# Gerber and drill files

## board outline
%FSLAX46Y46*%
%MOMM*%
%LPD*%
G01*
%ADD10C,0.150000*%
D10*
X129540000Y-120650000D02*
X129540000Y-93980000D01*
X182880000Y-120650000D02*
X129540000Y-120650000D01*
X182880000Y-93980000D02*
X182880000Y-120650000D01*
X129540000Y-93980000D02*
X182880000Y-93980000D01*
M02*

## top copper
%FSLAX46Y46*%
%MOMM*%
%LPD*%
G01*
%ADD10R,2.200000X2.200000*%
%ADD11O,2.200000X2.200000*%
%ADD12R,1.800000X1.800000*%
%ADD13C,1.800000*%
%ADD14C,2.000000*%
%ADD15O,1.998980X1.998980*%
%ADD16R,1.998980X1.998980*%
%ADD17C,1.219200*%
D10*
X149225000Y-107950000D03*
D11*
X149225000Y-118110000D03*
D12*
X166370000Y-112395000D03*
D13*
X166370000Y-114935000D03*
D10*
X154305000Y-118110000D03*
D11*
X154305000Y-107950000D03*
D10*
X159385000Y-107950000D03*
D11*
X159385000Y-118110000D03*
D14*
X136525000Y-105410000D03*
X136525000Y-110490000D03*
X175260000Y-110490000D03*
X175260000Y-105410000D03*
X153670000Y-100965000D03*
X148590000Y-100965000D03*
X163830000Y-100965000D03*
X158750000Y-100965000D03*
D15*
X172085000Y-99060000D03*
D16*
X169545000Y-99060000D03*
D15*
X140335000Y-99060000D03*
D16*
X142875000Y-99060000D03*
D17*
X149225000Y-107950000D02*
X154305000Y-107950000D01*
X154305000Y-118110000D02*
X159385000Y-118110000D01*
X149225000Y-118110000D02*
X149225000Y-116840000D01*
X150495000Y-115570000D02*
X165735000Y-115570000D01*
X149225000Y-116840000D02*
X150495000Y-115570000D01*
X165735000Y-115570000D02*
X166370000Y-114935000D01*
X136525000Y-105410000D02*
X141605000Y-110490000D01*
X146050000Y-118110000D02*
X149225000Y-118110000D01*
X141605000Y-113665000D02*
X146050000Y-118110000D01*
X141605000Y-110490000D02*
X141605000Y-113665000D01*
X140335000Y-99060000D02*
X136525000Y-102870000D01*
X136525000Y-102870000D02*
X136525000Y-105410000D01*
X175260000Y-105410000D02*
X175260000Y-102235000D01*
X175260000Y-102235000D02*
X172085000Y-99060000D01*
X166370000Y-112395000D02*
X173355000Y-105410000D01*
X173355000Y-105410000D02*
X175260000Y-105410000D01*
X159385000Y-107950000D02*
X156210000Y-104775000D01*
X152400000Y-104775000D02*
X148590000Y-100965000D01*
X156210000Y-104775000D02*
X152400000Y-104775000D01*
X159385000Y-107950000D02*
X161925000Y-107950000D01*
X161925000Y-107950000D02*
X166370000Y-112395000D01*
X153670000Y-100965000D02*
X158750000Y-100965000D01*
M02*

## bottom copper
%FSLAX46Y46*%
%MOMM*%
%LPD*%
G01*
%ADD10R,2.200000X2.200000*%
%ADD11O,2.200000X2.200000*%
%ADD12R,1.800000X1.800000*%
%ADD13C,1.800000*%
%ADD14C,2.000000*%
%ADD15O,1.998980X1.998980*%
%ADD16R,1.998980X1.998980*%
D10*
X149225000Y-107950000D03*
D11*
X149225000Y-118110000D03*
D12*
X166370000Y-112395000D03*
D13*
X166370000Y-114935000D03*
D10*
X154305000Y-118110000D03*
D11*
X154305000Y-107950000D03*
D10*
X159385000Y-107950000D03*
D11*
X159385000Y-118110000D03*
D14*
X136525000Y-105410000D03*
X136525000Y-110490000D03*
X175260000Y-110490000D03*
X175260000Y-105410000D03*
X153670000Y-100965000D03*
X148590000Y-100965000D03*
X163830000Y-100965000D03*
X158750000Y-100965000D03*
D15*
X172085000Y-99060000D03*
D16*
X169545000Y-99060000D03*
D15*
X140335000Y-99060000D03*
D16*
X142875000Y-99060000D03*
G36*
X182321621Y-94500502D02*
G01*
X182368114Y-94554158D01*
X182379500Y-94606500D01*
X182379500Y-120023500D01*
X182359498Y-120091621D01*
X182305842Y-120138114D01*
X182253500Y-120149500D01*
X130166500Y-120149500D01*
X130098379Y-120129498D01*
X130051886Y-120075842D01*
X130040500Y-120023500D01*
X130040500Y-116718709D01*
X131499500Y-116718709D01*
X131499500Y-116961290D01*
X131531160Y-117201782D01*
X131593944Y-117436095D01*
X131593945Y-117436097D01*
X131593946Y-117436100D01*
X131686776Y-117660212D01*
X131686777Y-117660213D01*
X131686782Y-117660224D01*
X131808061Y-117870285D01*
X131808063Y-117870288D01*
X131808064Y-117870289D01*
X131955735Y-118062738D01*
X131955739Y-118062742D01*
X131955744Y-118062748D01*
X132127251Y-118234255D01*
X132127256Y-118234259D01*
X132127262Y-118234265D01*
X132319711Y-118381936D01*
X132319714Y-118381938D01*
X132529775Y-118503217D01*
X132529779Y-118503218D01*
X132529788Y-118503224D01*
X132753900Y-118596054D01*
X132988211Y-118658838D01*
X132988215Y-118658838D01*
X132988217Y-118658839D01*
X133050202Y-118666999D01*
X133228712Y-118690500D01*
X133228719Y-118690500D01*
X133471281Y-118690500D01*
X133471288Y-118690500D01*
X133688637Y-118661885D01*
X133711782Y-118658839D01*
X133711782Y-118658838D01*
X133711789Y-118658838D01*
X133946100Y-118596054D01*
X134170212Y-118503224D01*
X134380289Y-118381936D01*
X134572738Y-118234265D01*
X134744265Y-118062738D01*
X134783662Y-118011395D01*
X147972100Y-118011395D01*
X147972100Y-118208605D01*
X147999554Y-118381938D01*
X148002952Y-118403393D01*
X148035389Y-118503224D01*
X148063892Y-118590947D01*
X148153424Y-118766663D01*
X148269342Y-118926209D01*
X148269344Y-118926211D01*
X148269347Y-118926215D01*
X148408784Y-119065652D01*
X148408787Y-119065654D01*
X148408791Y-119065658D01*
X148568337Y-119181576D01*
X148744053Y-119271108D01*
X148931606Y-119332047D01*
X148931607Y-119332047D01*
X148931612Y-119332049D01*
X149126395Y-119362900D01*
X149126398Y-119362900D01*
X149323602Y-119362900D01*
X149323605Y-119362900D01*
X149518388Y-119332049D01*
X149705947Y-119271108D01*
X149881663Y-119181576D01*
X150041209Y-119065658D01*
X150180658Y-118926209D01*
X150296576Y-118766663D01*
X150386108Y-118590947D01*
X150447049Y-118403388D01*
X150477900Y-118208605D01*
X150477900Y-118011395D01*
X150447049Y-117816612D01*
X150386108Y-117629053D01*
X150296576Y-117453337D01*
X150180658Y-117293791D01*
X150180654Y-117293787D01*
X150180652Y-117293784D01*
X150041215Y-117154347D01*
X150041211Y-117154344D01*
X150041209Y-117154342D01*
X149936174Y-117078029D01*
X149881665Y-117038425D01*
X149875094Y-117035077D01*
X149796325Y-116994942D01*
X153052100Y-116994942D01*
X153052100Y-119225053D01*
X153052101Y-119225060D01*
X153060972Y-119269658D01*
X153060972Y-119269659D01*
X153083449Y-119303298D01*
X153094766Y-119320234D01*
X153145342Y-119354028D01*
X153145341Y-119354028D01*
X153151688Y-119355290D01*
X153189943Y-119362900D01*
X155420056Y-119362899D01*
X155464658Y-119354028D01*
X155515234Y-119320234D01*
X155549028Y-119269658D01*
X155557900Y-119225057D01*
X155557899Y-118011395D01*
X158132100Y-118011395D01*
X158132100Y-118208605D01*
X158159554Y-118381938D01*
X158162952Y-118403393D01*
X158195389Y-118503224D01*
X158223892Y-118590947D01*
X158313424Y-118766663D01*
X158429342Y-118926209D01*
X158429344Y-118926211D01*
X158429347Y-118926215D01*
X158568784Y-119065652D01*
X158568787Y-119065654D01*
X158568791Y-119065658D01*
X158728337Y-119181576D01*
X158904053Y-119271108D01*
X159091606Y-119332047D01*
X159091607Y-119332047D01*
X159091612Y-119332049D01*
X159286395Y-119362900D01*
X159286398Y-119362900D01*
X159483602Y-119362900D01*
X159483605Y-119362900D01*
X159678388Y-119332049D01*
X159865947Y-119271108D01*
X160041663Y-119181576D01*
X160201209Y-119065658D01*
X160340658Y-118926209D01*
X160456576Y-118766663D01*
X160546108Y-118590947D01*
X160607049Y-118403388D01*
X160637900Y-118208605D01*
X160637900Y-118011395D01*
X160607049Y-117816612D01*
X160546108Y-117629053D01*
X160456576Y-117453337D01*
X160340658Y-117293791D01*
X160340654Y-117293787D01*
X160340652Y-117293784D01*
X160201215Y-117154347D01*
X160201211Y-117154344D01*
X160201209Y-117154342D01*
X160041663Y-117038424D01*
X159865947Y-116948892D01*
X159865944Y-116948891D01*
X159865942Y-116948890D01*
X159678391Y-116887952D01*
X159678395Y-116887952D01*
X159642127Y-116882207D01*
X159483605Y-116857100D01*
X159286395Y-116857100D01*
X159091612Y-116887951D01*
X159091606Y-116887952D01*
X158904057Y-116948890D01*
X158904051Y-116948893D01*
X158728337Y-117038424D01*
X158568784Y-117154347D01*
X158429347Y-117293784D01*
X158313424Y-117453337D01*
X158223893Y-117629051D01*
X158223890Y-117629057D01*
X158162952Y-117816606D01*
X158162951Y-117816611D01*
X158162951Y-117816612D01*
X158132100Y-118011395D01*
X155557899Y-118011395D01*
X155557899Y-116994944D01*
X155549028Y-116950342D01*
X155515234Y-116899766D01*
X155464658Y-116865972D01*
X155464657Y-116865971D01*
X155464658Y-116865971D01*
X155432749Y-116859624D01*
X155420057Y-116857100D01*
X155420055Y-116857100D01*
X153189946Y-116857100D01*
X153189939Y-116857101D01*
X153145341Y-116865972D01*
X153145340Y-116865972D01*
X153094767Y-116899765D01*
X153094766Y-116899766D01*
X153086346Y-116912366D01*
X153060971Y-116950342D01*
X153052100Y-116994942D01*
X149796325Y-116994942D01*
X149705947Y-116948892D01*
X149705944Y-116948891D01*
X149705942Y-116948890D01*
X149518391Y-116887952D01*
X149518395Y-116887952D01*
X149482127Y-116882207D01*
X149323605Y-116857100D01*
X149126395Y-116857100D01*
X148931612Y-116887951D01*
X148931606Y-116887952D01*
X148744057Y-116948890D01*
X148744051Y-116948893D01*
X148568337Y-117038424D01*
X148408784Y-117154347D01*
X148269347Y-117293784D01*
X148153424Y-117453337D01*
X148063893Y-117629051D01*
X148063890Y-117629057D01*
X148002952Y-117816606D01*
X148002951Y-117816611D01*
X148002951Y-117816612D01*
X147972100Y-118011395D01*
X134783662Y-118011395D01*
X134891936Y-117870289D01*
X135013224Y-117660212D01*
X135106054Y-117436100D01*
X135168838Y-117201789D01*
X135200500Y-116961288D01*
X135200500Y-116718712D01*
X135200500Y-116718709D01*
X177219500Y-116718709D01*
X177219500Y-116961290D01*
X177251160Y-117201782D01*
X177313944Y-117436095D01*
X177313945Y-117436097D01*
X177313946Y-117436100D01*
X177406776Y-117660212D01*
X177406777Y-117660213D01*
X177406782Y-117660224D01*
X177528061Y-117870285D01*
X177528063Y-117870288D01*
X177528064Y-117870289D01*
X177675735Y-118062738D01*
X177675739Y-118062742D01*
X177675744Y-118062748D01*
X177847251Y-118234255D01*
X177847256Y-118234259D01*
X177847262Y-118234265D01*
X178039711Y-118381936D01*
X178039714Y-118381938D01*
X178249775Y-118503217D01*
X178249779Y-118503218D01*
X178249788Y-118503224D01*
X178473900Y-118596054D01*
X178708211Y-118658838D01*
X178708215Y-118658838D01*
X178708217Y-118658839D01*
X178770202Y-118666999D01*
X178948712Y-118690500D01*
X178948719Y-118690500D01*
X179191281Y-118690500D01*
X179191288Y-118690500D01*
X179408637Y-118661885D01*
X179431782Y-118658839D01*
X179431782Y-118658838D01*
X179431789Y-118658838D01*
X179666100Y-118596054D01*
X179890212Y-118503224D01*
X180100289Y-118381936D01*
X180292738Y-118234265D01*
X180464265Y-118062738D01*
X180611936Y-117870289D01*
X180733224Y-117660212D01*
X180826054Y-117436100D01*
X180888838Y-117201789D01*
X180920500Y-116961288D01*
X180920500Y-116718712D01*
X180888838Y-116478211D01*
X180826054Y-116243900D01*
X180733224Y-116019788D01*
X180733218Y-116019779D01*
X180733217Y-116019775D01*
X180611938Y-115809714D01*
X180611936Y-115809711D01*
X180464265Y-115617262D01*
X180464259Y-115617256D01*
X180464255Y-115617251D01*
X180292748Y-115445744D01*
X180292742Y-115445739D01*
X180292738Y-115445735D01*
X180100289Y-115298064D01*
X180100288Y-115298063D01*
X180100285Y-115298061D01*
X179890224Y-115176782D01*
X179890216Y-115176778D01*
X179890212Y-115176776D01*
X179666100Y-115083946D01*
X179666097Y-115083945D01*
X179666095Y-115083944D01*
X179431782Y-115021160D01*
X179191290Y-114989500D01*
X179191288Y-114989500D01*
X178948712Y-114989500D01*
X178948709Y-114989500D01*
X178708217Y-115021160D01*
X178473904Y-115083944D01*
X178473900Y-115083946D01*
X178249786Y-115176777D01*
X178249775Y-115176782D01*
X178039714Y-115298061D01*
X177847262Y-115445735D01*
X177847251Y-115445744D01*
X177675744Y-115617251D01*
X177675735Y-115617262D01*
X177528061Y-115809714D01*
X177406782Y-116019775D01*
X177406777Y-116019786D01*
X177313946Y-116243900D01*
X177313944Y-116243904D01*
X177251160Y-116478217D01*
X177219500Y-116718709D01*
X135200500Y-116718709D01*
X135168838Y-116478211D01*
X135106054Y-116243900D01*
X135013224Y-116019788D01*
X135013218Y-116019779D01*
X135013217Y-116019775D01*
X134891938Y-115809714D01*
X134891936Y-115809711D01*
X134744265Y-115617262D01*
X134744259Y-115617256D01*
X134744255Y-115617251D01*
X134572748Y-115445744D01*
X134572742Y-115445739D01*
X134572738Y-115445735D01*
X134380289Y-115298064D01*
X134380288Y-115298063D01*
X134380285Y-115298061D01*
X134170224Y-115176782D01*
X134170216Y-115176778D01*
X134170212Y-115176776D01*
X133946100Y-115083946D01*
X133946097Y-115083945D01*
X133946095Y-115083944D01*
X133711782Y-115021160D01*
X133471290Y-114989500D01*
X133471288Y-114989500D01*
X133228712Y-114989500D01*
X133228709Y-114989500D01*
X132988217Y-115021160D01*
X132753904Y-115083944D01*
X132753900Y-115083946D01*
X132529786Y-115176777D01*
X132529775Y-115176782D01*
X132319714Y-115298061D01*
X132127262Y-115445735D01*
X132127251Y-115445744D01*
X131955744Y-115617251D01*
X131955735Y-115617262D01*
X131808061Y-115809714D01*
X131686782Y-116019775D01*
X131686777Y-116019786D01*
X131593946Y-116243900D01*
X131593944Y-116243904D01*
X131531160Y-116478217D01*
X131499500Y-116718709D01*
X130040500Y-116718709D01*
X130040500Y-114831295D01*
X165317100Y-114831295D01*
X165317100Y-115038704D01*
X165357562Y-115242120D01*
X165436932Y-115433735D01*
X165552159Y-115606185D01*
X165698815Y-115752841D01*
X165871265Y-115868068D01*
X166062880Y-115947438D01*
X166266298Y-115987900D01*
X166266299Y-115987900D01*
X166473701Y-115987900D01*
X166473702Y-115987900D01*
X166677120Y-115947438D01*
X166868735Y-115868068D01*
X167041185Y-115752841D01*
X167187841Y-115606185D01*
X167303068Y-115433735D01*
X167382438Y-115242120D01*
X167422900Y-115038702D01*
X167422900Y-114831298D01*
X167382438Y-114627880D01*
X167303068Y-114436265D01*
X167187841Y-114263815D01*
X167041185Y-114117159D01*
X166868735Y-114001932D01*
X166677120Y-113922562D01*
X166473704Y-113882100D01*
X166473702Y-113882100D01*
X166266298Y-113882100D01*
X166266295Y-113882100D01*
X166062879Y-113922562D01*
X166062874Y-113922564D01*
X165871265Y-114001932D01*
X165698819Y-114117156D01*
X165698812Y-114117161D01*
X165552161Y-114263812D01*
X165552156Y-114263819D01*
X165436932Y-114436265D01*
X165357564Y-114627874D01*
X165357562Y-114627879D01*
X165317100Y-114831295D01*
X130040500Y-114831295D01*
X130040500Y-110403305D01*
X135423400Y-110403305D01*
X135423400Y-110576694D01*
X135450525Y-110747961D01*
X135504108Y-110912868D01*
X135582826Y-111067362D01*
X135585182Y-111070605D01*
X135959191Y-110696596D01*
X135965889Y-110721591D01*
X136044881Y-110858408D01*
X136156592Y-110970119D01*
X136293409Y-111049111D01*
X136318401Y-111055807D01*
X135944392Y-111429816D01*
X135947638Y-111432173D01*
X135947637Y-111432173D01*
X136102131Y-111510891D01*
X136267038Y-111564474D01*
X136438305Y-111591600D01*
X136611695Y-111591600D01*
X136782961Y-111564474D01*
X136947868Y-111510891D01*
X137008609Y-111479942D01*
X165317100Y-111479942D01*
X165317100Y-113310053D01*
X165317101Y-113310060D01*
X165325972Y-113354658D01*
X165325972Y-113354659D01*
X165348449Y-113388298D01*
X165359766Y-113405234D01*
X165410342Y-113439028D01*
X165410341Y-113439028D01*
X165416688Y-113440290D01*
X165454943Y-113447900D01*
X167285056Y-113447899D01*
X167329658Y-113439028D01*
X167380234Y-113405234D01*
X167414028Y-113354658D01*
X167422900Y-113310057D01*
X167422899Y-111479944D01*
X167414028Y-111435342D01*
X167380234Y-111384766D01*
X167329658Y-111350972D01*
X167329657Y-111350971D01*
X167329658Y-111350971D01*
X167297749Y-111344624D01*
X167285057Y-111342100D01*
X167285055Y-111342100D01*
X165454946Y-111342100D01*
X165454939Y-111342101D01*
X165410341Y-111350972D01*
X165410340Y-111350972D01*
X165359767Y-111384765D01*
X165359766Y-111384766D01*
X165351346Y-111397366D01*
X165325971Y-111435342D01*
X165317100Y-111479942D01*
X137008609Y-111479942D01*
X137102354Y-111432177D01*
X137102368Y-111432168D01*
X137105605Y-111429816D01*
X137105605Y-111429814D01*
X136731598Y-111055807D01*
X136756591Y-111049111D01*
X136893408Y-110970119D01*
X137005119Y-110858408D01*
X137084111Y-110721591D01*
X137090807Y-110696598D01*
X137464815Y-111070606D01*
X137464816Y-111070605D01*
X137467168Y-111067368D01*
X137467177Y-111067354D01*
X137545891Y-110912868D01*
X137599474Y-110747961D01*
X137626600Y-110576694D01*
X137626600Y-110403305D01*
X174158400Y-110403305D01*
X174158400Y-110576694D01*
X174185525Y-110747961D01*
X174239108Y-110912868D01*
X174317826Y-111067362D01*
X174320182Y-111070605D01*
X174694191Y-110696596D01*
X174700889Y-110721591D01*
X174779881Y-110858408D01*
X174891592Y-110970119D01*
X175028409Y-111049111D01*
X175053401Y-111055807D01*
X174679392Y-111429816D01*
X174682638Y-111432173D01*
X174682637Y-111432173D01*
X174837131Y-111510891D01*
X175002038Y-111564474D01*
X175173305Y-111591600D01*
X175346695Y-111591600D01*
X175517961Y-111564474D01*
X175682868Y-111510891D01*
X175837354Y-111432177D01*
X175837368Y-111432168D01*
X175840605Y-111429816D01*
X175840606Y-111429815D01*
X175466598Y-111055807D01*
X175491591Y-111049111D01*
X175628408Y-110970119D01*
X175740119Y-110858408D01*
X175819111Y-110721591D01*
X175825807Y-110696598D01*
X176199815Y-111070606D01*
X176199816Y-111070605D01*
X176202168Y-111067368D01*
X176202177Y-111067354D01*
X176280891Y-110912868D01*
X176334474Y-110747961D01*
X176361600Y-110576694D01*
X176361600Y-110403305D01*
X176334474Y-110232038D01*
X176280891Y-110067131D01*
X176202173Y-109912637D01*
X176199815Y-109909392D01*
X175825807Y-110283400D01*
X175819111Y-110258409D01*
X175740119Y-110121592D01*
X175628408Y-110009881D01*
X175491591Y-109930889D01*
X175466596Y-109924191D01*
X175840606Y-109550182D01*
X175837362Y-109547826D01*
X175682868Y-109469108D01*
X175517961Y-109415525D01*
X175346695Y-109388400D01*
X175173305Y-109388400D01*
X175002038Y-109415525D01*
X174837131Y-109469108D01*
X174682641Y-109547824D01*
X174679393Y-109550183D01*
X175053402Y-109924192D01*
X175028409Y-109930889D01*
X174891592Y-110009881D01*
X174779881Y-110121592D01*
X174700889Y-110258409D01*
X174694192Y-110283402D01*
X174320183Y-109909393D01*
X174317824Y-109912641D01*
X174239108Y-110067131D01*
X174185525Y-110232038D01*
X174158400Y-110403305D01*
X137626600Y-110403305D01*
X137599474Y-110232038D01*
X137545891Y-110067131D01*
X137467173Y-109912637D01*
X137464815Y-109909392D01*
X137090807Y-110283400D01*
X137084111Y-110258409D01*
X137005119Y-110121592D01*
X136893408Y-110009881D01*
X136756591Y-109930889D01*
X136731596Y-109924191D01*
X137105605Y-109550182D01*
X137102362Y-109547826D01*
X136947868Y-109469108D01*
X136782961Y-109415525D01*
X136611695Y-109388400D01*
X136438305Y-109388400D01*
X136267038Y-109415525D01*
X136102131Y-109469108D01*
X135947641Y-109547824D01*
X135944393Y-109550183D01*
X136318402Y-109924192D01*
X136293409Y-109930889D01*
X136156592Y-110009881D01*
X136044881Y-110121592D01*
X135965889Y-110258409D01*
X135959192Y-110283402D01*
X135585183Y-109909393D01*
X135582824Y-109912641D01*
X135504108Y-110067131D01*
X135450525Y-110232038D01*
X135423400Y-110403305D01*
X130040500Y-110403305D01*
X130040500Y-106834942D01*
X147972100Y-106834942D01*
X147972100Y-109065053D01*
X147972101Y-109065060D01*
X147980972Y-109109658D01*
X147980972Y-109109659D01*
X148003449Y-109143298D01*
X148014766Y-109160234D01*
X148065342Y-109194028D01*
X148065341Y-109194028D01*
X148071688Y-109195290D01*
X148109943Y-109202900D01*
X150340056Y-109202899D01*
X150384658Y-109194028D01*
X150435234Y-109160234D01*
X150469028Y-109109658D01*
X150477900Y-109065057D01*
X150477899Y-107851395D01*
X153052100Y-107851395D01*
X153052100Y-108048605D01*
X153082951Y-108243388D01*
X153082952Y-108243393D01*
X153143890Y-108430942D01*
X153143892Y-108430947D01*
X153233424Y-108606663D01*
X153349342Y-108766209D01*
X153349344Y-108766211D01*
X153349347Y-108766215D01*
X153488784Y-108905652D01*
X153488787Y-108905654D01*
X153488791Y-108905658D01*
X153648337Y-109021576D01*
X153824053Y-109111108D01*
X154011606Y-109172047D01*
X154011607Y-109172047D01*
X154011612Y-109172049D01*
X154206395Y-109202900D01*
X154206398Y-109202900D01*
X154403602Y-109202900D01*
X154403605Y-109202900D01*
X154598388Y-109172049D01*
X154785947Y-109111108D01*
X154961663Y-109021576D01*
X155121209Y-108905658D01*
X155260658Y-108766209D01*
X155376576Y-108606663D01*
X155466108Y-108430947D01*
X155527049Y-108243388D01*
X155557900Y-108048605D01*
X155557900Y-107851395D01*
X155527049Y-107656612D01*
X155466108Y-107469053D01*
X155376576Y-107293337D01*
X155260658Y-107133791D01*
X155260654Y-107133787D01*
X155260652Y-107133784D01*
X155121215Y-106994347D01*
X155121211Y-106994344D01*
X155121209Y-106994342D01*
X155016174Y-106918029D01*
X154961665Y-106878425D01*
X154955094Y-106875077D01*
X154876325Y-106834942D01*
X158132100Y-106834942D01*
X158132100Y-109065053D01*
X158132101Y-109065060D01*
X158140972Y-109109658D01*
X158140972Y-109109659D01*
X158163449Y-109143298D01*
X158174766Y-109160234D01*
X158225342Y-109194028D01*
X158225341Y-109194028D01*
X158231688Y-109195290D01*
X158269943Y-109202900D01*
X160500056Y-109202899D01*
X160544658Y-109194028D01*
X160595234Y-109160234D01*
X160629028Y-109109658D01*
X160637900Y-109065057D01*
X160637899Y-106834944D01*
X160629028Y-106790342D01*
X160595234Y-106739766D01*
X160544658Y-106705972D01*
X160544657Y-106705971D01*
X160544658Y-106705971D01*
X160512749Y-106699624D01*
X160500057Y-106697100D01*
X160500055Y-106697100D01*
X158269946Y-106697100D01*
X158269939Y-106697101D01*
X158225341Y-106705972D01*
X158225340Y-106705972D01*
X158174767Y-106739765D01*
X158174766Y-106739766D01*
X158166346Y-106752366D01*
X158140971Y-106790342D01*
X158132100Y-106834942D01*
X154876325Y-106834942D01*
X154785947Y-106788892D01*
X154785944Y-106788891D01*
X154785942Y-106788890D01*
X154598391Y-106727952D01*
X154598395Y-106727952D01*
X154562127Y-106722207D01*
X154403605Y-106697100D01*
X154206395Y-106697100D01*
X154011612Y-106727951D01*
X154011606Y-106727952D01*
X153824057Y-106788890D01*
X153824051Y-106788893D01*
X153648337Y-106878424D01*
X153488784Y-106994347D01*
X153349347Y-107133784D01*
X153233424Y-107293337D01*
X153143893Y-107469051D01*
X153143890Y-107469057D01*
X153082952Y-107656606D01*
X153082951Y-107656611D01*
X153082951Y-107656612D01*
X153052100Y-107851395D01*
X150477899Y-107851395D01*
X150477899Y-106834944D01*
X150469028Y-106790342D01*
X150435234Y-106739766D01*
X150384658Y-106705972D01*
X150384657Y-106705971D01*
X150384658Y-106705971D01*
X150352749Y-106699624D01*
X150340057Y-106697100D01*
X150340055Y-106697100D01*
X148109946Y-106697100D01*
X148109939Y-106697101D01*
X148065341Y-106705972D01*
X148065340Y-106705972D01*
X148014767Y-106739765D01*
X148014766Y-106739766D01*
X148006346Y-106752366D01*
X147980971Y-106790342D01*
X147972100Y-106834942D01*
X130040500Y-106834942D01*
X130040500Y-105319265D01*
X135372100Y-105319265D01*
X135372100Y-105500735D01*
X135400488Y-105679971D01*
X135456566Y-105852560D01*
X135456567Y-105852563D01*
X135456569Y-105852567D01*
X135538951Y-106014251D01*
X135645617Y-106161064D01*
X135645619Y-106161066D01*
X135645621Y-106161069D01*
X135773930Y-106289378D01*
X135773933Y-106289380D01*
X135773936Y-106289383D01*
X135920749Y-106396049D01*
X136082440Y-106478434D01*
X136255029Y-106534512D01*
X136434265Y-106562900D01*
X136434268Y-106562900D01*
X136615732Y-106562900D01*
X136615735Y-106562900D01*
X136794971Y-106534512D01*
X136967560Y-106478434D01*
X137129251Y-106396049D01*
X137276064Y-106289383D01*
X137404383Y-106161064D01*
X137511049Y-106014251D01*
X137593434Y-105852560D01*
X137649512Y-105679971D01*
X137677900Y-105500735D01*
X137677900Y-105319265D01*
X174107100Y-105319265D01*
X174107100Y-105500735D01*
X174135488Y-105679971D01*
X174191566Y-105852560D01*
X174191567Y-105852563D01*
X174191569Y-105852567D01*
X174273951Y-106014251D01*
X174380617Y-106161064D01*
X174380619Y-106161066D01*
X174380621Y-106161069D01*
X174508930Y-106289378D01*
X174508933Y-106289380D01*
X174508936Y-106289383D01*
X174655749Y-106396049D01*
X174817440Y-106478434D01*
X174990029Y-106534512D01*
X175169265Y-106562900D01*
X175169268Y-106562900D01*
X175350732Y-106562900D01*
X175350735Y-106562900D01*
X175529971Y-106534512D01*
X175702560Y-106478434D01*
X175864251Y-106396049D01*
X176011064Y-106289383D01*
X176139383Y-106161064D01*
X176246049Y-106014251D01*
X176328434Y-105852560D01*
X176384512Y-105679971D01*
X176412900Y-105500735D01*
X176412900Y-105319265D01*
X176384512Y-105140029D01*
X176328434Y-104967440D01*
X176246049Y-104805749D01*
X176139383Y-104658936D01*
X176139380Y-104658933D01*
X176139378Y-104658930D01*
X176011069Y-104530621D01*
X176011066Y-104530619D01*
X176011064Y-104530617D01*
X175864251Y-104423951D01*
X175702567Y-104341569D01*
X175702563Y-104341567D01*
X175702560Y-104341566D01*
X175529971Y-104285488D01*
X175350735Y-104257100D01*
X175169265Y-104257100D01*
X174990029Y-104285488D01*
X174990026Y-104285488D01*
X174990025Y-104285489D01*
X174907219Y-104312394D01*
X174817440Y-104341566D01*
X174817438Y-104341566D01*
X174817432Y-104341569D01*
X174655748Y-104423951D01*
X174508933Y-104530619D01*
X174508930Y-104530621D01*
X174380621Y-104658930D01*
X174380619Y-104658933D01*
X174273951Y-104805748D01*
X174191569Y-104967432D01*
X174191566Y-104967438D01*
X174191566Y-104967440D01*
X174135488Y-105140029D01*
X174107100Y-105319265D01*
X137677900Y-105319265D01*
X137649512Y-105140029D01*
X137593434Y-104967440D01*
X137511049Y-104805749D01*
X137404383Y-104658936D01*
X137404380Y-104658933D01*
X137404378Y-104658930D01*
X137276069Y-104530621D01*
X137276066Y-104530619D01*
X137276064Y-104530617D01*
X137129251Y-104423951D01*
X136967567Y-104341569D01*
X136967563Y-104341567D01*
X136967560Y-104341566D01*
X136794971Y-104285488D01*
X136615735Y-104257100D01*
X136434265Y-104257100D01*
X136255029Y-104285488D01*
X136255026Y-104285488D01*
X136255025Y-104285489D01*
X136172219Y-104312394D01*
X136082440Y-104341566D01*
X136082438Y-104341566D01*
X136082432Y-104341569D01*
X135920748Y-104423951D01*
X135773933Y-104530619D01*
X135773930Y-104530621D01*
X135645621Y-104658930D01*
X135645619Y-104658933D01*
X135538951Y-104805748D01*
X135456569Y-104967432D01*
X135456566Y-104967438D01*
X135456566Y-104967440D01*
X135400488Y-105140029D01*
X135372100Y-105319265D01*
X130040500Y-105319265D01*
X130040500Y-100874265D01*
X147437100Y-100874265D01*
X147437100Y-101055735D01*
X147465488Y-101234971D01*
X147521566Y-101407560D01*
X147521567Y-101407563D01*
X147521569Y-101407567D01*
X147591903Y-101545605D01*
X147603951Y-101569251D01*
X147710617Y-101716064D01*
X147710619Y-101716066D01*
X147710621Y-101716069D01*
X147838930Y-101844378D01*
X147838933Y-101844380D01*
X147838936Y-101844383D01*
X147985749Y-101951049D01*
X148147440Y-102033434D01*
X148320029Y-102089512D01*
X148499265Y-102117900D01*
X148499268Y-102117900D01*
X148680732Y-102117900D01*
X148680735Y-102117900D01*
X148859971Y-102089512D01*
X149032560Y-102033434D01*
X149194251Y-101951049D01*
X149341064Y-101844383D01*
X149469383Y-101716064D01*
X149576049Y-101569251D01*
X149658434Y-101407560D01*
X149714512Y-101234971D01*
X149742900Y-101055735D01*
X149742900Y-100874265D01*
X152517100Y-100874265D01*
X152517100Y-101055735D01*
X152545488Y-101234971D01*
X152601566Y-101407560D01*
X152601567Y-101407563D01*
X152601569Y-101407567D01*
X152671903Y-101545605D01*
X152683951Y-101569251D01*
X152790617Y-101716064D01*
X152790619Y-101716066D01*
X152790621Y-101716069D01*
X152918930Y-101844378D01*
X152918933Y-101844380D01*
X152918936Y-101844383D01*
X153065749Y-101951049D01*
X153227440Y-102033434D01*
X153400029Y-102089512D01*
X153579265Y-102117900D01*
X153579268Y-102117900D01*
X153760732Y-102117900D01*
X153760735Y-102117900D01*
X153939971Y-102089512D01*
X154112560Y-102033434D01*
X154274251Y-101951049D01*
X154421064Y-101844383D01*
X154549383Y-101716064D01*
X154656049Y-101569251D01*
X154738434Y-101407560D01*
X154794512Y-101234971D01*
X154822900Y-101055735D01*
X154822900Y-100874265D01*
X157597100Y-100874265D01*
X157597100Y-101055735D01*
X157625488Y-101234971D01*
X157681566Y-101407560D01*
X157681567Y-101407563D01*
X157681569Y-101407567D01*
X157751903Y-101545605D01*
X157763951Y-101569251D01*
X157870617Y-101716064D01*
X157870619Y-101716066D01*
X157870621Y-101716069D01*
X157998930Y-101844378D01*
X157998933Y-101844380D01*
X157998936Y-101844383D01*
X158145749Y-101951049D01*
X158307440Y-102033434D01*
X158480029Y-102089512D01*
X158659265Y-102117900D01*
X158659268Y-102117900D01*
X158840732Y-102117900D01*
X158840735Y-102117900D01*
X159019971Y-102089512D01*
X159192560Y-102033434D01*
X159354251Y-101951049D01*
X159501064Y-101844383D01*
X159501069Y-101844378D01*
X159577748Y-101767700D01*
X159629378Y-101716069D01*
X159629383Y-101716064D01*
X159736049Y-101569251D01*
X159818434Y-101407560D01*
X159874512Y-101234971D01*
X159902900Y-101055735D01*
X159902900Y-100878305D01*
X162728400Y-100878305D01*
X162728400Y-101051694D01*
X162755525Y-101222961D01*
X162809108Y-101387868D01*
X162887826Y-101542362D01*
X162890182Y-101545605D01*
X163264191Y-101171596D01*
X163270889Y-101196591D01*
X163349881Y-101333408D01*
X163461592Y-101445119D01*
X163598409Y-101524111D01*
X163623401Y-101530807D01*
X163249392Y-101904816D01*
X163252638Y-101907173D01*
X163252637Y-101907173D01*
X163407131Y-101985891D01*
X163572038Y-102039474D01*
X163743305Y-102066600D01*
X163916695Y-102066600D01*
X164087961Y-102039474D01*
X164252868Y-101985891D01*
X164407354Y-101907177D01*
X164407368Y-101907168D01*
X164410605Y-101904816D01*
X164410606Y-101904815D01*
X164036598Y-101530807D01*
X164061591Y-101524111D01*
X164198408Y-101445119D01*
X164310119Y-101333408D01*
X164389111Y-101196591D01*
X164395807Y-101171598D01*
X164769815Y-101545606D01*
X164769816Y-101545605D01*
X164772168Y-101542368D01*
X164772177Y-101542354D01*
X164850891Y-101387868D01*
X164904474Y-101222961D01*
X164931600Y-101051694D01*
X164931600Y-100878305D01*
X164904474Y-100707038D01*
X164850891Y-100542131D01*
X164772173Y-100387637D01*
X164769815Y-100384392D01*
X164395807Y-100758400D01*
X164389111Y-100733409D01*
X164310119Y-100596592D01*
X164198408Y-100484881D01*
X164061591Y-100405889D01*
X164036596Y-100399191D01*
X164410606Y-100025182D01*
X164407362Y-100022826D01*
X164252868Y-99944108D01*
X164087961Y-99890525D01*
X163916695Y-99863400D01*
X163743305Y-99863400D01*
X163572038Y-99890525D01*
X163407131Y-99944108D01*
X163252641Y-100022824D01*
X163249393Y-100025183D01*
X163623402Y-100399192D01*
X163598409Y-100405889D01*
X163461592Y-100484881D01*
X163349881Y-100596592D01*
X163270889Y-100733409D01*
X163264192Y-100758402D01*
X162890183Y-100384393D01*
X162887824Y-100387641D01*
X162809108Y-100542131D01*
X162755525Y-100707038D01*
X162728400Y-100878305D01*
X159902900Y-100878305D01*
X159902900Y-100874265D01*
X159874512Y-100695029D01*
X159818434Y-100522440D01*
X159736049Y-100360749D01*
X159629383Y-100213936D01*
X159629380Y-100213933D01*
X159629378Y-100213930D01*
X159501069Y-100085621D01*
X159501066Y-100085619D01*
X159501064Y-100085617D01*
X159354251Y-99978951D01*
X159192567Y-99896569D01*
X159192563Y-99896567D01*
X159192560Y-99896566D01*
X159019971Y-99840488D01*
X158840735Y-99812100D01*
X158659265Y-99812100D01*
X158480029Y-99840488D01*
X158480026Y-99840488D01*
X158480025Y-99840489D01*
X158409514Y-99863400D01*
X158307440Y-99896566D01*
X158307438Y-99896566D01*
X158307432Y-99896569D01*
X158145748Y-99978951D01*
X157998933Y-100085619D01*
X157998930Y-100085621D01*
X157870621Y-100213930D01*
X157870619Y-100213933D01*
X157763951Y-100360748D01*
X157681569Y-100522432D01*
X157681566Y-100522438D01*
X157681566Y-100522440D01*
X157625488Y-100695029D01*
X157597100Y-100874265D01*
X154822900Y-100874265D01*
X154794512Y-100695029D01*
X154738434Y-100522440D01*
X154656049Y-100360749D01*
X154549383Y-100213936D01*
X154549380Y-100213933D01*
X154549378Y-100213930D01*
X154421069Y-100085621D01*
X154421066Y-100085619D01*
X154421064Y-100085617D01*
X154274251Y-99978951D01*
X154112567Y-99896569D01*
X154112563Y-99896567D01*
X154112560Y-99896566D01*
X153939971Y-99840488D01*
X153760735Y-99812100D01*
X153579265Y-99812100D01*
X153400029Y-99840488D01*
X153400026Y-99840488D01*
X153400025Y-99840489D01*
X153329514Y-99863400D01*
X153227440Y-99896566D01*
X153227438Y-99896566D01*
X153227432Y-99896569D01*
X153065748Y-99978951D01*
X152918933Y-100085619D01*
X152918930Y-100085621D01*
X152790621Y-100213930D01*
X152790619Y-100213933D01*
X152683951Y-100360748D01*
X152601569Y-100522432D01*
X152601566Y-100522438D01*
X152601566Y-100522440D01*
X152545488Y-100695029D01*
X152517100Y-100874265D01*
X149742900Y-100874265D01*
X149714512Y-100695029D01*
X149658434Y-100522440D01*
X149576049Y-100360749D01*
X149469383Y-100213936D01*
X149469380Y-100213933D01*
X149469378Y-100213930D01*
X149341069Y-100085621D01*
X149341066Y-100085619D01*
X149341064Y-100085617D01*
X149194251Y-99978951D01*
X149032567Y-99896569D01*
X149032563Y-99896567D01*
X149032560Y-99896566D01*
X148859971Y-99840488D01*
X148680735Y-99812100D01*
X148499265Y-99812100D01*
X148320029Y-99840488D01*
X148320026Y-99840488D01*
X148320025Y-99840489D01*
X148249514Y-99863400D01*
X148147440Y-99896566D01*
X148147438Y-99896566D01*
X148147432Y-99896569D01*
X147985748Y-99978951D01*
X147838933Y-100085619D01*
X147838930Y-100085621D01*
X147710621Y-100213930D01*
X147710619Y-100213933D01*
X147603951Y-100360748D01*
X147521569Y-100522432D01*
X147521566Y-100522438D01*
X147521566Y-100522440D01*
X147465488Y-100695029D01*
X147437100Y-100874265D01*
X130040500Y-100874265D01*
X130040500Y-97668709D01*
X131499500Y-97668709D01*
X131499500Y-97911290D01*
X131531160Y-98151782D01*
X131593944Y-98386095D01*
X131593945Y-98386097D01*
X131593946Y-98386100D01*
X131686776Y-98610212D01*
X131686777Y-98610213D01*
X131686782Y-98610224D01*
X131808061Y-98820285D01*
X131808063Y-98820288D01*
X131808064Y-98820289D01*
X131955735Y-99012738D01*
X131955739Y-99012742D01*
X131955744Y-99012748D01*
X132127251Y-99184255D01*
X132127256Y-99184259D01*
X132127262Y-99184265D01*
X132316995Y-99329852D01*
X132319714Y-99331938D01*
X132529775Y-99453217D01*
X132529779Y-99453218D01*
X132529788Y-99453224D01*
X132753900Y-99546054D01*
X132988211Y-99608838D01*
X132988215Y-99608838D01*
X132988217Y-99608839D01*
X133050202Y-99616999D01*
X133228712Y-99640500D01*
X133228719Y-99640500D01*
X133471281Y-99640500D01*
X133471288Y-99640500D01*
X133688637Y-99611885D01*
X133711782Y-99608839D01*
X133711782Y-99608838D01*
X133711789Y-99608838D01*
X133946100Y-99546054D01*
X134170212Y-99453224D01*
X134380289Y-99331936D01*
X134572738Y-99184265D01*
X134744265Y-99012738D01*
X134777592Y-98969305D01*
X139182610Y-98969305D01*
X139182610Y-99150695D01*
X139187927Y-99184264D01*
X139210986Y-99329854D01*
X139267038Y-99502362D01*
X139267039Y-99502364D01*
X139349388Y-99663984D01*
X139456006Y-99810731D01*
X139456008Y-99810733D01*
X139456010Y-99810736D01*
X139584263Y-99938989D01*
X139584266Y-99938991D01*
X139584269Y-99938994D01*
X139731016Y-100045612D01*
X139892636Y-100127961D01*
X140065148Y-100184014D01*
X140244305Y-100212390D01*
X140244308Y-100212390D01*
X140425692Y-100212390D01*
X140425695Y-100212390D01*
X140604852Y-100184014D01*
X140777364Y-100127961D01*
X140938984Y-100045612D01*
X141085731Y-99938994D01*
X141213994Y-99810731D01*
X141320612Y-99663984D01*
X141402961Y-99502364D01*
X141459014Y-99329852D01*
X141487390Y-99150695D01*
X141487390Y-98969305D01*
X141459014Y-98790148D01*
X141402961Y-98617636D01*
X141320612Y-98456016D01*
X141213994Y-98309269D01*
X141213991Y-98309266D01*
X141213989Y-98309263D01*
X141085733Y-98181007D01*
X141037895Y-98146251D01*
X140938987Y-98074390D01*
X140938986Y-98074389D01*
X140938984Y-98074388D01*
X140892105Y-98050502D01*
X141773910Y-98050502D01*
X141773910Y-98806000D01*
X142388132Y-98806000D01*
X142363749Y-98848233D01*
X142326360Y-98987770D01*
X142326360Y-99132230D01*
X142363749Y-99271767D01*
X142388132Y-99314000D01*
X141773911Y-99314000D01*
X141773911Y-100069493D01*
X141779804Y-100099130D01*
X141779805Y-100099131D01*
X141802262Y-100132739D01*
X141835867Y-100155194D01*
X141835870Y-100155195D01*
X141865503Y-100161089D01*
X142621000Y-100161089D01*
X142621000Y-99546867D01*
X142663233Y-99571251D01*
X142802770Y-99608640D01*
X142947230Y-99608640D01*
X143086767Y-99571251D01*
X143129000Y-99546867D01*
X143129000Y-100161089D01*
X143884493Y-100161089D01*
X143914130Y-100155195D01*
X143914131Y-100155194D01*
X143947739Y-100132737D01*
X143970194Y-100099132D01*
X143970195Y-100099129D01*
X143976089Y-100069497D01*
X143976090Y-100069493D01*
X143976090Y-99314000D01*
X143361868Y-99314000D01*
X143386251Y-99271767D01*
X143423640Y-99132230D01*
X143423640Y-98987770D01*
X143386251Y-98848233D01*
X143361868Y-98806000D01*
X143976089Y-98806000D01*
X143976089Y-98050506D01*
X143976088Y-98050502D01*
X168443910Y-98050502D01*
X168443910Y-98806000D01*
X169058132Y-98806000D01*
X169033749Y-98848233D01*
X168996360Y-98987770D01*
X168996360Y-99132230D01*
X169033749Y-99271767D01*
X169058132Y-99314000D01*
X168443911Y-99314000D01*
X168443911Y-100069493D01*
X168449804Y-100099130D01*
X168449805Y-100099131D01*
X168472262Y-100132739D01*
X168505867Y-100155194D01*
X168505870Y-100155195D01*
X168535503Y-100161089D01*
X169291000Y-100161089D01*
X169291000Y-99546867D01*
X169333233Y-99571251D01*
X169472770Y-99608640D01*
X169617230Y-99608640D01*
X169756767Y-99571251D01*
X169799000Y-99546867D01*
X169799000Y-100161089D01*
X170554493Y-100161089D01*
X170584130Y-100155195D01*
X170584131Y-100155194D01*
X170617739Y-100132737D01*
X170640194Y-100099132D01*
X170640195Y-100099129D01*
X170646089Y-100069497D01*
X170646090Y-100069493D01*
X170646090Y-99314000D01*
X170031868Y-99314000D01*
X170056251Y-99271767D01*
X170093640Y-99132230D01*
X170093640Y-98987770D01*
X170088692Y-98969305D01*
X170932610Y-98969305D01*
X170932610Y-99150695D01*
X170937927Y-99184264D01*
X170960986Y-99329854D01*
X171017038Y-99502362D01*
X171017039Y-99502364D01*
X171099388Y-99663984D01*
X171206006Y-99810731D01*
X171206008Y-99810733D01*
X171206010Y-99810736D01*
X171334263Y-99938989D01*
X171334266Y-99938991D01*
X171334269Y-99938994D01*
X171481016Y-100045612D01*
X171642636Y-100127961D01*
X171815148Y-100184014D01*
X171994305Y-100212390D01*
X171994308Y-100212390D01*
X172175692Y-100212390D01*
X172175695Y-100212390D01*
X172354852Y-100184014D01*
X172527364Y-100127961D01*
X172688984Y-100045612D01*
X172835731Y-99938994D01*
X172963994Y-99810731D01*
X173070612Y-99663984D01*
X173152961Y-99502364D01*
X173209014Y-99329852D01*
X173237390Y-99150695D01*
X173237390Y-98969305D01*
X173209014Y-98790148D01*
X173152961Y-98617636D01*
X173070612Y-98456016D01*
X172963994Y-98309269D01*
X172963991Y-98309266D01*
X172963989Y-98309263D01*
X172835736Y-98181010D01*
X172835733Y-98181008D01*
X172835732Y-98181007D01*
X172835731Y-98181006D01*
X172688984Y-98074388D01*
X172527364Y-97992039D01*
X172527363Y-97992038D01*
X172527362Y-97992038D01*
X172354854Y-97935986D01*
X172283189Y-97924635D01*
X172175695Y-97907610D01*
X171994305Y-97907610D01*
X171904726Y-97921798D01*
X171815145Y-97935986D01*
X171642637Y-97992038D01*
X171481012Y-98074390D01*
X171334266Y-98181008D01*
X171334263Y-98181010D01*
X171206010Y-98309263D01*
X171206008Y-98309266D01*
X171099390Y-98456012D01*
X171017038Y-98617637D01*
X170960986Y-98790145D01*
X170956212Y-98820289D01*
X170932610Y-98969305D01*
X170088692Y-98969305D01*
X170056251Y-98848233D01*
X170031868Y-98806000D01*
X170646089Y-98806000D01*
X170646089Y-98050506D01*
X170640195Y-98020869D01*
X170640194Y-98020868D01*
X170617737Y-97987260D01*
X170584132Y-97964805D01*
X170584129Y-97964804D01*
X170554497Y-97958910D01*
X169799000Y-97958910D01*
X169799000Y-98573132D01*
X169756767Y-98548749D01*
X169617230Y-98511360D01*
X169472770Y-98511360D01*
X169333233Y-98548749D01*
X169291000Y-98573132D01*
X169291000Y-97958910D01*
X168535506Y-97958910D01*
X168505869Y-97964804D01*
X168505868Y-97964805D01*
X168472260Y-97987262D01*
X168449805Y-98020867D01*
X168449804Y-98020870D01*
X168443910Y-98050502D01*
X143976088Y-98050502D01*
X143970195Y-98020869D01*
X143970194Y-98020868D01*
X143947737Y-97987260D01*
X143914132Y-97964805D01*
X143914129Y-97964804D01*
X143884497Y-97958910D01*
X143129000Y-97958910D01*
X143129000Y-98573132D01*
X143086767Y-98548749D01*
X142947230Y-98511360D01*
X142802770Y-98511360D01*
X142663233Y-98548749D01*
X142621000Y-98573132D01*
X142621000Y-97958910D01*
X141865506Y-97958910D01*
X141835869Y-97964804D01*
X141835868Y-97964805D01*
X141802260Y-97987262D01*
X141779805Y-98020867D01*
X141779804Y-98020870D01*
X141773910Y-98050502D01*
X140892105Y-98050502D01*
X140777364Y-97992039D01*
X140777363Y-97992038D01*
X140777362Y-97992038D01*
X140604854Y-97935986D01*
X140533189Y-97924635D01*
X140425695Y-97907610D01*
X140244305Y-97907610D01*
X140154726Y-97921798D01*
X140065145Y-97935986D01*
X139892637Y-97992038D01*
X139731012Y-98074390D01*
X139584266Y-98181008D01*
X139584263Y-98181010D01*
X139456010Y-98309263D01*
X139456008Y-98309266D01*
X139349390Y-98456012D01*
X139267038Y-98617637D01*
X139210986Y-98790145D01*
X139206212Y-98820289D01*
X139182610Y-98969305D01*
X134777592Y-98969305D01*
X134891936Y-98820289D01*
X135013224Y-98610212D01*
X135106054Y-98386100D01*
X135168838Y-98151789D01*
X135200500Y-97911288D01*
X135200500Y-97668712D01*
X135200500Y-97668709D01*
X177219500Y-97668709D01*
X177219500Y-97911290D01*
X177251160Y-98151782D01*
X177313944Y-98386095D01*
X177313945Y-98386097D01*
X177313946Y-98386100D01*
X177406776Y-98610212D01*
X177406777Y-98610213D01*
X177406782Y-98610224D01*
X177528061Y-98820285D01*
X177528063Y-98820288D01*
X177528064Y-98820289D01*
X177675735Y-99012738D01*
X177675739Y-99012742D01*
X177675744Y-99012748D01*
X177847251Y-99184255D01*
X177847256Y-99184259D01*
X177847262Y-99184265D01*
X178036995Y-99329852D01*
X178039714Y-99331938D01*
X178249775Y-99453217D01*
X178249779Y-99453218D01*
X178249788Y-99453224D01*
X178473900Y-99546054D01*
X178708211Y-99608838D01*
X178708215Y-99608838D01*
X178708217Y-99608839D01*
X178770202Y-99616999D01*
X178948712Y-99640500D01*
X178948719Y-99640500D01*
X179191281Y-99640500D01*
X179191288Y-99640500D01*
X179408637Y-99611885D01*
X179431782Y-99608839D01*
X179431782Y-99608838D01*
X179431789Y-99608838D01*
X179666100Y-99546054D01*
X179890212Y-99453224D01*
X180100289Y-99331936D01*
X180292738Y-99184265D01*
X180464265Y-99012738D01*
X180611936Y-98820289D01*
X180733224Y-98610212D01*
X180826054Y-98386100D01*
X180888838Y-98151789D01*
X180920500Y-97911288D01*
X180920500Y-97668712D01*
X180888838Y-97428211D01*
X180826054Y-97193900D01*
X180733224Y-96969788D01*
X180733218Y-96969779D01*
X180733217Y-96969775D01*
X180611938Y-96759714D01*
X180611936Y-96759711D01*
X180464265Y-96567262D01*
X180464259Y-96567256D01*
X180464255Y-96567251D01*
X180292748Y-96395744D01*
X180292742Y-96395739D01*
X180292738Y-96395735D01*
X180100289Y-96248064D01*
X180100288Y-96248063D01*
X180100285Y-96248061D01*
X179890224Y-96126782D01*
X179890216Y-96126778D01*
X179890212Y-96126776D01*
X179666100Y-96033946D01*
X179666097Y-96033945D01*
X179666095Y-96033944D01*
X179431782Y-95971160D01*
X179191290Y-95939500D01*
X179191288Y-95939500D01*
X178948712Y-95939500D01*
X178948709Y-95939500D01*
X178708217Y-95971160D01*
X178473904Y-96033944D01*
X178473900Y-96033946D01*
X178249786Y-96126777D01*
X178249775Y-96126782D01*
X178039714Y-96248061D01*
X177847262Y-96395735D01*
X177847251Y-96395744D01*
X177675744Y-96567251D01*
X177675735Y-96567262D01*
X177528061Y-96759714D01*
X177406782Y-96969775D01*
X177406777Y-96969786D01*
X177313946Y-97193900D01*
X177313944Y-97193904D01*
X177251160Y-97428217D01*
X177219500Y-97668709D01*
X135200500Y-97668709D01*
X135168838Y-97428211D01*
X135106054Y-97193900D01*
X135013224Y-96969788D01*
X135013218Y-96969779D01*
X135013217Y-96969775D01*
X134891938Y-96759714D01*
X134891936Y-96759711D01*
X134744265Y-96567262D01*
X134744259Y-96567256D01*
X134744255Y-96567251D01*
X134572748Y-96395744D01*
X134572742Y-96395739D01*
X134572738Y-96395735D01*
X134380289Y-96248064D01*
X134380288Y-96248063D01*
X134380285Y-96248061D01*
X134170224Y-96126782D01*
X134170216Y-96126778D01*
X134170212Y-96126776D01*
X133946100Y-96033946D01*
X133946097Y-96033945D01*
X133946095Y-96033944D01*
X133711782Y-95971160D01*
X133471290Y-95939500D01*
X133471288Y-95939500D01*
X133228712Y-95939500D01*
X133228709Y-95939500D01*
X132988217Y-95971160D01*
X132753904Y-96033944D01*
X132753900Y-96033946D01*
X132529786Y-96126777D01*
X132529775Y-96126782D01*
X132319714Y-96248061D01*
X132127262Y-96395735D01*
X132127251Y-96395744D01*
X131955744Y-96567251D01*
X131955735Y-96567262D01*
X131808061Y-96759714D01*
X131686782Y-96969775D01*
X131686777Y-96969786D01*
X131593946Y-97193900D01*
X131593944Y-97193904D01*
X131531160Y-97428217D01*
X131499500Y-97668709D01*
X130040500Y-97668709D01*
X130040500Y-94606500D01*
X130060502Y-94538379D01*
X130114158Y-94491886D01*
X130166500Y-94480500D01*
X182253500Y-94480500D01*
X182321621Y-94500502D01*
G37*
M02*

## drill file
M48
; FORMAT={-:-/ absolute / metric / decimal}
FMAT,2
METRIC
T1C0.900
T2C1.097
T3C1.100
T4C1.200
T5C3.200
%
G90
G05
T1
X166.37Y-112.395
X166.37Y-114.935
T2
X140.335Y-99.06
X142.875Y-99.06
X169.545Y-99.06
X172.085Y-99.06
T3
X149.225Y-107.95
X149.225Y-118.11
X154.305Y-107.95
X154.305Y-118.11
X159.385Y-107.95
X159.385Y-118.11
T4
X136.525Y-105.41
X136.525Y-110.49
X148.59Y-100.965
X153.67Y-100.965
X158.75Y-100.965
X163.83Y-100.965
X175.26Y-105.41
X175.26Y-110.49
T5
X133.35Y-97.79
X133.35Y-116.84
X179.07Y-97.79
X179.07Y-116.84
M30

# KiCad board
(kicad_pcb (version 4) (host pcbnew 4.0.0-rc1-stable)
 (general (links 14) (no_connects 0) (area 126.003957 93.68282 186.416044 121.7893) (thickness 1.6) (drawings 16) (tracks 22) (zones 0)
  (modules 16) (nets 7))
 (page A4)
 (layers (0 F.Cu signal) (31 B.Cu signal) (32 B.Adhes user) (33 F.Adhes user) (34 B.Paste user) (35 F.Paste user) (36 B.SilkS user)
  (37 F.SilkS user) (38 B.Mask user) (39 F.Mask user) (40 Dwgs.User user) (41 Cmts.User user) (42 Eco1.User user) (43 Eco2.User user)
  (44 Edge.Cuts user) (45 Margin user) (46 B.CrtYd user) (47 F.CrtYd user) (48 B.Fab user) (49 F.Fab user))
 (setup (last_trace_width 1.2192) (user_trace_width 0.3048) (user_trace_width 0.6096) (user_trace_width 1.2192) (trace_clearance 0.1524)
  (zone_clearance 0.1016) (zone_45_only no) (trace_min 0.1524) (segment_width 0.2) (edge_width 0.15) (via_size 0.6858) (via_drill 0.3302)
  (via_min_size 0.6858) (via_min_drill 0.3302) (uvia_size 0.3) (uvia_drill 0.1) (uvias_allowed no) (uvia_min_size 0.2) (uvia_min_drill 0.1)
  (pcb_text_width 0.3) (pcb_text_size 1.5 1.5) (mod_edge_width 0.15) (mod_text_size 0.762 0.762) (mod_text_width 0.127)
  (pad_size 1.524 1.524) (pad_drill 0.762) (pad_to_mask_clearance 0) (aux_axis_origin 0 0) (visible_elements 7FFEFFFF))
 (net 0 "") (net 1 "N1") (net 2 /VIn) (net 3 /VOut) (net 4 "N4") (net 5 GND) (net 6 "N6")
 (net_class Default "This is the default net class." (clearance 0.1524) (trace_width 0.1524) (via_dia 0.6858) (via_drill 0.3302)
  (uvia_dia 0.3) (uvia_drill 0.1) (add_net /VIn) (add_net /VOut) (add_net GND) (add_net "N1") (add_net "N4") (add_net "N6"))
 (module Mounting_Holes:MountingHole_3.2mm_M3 (layer F.Cu) (at 179.07 97.79)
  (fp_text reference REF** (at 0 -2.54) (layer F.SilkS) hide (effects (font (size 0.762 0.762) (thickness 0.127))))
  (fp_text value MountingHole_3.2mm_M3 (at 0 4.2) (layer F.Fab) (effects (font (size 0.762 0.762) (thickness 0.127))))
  (pad 1 np_thru_hole circle (at 0 0) (size 3.2 3.2) (drill 3.2) (layers *.Cu *.Mask)))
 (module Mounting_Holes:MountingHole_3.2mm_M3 (layer F.Cu) (at 179.07 116.84)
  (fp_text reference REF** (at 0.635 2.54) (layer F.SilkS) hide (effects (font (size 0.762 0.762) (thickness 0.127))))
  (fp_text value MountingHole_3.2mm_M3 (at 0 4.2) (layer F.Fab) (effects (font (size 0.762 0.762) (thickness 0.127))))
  (pad 1 np_thru_hole circle (at 0 0) (size 3.2 3.2) (drill 3.2) (layers *.Cu *.Mask)))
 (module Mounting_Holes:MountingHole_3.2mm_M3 (layer F.Cu) (at 133.35 116.84)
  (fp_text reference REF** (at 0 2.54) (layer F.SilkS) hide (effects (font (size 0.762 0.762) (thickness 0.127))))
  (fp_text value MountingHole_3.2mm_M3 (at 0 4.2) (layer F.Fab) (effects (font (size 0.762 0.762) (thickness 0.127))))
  (pad 1 np_thru_hole circle (at 0 0) (size 3.2 3.2) (drill 3.2) (layers *.Cu *.Mask)))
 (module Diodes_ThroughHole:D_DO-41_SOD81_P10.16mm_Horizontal (layer F.Cu) (at 149.225 107.95 270)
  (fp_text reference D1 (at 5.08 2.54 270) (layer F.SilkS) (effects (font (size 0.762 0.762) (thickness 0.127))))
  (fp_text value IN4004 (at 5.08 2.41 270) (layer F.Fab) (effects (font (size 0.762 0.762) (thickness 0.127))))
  (pad 1 thru_hole rect (at 0 0 270) (size 2.2 2.2) (drill 1.1) (layers *.Cu *.Mask) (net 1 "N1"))
  (pad 2 thru_hole oval (at 10.16 0 270) (size 2.2 2.2) (drill 1.1) (layers *.Cu *.Mask) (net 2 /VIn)))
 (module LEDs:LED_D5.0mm (layer B.Cu) (at 166.37 112.395 270)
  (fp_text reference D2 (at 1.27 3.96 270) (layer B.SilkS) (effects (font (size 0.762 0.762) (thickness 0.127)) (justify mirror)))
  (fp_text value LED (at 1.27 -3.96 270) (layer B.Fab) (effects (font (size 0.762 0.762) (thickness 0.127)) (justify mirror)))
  (pad 1 thru_hole rect (at 0 0 270) (size 1.8 1.8) (drill 0.9) (layers *.Cu *.Mask) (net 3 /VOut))
  (pad 2 thru_hole circle (at 2.54 0 270) (size 1.8 1.8) (drill 0.9) (layers *.Cu *.Mask) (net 2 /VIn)))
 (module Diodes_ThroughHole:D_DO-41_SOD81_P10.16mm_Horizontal (layer F.Cu) (at 154.305 118.11 90)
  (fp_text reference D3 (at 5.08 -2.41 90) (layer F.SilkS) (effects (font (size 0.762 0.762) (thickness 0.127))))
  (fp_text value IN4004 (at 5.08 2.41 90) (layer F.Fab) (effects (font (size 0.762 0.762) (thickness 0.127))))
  (pad 1 thru_hole rect (at 0 0 90) (size 2.2 2.2) (drill 1.1) (layers *.Cu *.Mask) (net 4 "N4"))
  (pad 2 thru_hole oval (at 10.16 0 90) (size 2.2 2.2) (drill 1.1) (layers *.Cu *.Mask) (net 1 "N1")))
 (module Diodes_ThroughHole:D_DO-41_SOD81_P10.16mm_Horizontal (layer F.Cu) (at 159.385 107.95 270)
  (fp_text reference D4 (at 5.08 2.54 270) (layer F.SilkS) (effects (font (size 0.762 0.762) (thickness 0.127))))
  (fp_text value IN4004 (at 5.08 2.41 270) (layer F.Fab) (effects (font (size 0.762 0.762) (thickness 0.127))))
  (pad 1 thru_hole rect (at 0 0 270) (size 2.2 2.2) (drill 1.1) (layers *.Cu *.Mask) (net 3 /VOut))
  (pad 2 thru_hole oval (at 10.16 0 270) (size 2.2 2.2) (drill 1.1) (layers *.Cu *.Mask) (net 4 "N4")))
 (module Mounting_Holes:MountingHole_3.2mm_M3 (layer F.Cu) (at 133.35 97.79)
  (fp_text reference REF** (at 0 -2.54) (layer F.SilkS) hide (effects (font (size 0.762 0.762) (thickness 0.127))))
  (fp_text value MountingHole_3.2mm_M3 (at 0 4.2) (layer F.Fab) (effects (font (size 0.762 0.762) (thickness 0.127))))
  (pad 1 np_thru_hole circle (at 0 0) (size 3.2 3.2) (drill 3.2) (layers *.Cu *.Mask)))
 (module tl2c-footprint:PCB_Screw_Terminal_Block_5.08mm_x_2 (layer F.Cu) (at 136.525 105.41 270)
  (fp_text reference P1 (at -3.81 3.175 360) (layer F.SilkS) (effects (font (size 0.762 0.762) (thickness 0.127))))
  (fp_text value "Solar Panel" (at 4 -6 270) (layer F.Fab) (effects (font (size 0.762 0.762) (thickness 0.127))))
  (pad 1 thru_hole circle (at 0 0 270) (size 2 2) (drill 1.2) (layers *.Cu *.Mask F.SilkS) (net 2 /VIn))
  (pad 2 thru_hole circle (at 5.08 0 270) (size 2 2) (drill 1.2) (layers *.Cu *.Mask F.SilkS) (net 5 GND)))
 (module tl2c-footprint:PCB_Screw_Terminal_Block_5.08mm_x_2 (layer F.Cu) (at 175.26 110.49 90)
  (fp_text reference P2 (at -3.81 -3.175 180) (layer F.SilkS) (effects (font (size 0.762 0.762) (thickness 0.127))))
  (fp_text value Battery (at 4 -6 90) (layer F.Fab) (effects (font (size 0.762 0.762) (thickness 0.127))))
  (pad 1 thru_hole circle (at 0 0 90) (size 2 2) (drill 1.2) (layers *.Cu *.Mask F.SilkS) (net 5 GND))
  (pad 2 thru_hole circle (at 5.08 0 90) (size 2 2) (drill 1.2) (layers *.Cu *.Mask F.SilkS) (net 3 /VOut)))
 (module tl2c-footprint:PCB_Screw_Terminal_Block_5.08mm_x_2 (layer F.Cu) (at 153.67 100.965 180)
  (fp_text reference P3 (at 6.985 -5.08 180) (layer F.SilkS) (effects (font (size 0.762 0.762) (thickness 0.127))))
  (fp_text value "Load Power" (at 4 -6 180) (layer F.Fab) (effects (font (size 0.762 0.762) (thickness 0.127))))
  (pad 1 thru_hole circle (at 0 0 180) (size 2 2) (drill 1.2) (layers *.Cu *.Mask F.SilkS) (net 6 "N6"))
  (pad 2 thru_hole circle (at 5.08 0 180) (size 2 2) (drill 1.2) (layers *.Cu *.Mask F.SilkS) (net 3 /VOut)))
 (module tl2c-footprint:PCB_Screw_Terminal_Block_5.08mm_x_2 (layer F.Cu) (at 163.83 100.965 180)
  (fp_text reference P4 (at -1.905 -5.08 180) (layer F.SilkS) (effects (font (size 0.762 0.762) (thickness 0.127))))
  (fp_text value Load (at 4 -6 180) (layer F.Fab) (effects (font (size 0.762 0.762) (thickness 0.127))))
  (pad 1 thru_hole circle (at 0 0 180) (size 2 2) (drill 1.2) (layers *.Cu *.Mask F.SilkS) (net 5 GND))
  (pad 2 thru_hole circle (at 5.08 0 180) (size 2 2) (drill 1.2) (layers *.Cu *.Mask F.SilkS) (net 6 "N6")))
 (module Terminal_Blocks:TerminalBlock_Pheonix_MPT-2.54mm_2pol (layer F.Cu) (at 169.545 99.06)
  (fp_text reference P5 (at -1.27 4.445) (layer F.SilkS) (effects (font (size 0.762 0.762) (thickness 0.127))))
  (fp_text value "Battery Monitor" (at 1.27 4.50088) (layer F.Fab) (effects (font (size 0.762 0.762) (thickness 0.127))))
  (pad 2 thru_hole oval (at 2.54 0) (size 1.99898 1.99898) (drill 1.09728) (layers *.Cu *.Mask) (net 3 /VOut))
  (pad 1 thru_hole rect (at 0 0) (size 1.99898 1.99898) (drill 1.09728) (layers *.Cu *.Mask) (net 5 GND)))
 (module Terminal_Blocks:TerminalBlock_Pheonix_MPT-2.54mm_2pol (layer F.Cu) (at 142.875 99.06 180)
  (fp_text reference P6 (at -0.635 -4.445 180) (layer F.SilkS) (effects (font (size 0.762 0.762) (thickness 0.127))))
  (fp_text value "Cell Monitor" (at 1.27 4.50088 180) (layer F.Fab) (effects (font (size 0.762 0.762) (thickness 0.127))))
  (pad 2 thru_hole oval (at 2.54 0 180) (size 1.99898 1.99898) (drill 1.09728) (layers *.Cu *.Mask) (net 2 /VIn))
  (pad 1 thru_hole rect (at 0 0 180) (size 1.99898 1.99898) (drill 1.09728) (layers *.Cu *.Mask) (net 5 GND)))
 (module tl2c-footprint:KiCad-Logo (layer F.Cu) (at 167.64 118.11)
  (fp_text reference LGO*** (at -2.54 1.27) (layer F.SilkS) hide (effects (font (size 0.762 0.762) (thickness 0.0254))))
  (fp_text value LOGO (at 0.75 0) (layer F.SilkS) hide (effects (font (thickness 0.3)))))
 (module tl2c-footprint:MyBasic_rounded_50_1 (layer F.Cu) (at 141.605 116.84)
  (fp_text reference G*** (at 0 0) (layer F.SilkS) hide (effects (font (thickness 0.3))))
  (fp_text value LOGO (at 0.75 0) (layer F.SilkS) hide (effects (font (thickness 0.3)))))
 (gr_line (start 129.54 120.65) (end 129.54 93.98) (angle 90) (layer Edge.Cuts) (width 0.15))
 (gr_line (start 182.88 120.65) (end 129.54 120.65) (angle 90) (layer Edge.Cuts) (width 0.15))
 (gr_line (start 182.88 93.98) (end 182.88 120.65) (angle 90) (layer Edge.Cuts) (width 0.15))
 (gr_line (start 129.54 93.98) (end 182.88 93.98) (angle 90) (layer Edge.Cuts) (width 0.15))
 (segment (start 149.225 107.95) (end 154.305 107.95) (width 1.2192) (layer F.Cu) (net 1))
 (segment (start 154.305 118.11) (end 159.385 118.11) (width 1.2192) (layer F.Cu) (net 4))
 (segment (start 149.225 118.11) (end 149.225 116.84) (width 1.2192) (layer F.Cu) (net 2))
 (segment (start 150.495 115.57) (end 165.735 115.57) (width 1.2192) (layer F.Cu) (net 2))
 (segment (start 149.225 116.84) (end 150.495 115.57) (width 1.2192) (layer F.Cu) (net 2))
 (segment (start 165.735 115.57) (end 166.37 114.935) (width 1.2192) (layer F.Cu) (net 2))
 (segment (start 136.525 105.41) (end 141.605 110.49) (width 1.2192) (layer F.Cu) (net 2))
 (segment (start 146.05 118.11) (end 149.225 118.11) (width 1.2192) (layer F.Cu) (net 2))
 (segment (start 141.605 113.665) (end 146.05 118.11) (width 1.2192) (layer F.Cu) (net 2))
 (segment (start 141.605 110.49) (end 141.605 113.665) (width 1.2192) (layer F.Cu) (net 2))
 (segment (start 140.335 99.06) (end 136.525 102.87) (width 1.2192) (layer F.Cu) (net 2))
 (segment (start 136.525 102.87) (end 136.525 105.41) (width 1.2192) (layer F.Cu) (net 2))
 (segment (start 175.26 105.41) (end 175.26 102.235) (width 1.2192) (layer F.Cu) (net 3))
 (segment (start 175.26 102.235) (end 172.085 99.06) (width 1.2192) (layer F.Cu) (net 3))
 (segment (start 166.37 112.395) (end 173.355 105.41) (width 1.2192) (layer F.Cu) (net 3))
 (segment (start 173.355 105.41) (end 175.26 105.41) (width 1.2192) (layer F.Cu) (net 3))
 (segment (start 159.385 107.95) (end 156.21 104.775) (width 1.2192) (layer F.Cu) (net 3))
 (segment (start 152.4 104.775) (end 148.59 100.965) (width 1.2192) (layer F.Cu) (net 3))
 (segment (start 156.21 104.775) (end 152.4 104.775) (width 1.2192) (layer F.Cu) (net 3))
 (segment (start 159.385 107.95) (end 161.925 107.95) (width 1.2192) (layer F.Cu) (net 3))
 (segment (start 161.925 107.95) (end 166.37 112.395) (width 1.2192) (layer F.Cu) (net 3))
 (segment (start 153.67 100.965) (end 158.75 100.965) (width 1.2192) (layer F.Cu) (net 6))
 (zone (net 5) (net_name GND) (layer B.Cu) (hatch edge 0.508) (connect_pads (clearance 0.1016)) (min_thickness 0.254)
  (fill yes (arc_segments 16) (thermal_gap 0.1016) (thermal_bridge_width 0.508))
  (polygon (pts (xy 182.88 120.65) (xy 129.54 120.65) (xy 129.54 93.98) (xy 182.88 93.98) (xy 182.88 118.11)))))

